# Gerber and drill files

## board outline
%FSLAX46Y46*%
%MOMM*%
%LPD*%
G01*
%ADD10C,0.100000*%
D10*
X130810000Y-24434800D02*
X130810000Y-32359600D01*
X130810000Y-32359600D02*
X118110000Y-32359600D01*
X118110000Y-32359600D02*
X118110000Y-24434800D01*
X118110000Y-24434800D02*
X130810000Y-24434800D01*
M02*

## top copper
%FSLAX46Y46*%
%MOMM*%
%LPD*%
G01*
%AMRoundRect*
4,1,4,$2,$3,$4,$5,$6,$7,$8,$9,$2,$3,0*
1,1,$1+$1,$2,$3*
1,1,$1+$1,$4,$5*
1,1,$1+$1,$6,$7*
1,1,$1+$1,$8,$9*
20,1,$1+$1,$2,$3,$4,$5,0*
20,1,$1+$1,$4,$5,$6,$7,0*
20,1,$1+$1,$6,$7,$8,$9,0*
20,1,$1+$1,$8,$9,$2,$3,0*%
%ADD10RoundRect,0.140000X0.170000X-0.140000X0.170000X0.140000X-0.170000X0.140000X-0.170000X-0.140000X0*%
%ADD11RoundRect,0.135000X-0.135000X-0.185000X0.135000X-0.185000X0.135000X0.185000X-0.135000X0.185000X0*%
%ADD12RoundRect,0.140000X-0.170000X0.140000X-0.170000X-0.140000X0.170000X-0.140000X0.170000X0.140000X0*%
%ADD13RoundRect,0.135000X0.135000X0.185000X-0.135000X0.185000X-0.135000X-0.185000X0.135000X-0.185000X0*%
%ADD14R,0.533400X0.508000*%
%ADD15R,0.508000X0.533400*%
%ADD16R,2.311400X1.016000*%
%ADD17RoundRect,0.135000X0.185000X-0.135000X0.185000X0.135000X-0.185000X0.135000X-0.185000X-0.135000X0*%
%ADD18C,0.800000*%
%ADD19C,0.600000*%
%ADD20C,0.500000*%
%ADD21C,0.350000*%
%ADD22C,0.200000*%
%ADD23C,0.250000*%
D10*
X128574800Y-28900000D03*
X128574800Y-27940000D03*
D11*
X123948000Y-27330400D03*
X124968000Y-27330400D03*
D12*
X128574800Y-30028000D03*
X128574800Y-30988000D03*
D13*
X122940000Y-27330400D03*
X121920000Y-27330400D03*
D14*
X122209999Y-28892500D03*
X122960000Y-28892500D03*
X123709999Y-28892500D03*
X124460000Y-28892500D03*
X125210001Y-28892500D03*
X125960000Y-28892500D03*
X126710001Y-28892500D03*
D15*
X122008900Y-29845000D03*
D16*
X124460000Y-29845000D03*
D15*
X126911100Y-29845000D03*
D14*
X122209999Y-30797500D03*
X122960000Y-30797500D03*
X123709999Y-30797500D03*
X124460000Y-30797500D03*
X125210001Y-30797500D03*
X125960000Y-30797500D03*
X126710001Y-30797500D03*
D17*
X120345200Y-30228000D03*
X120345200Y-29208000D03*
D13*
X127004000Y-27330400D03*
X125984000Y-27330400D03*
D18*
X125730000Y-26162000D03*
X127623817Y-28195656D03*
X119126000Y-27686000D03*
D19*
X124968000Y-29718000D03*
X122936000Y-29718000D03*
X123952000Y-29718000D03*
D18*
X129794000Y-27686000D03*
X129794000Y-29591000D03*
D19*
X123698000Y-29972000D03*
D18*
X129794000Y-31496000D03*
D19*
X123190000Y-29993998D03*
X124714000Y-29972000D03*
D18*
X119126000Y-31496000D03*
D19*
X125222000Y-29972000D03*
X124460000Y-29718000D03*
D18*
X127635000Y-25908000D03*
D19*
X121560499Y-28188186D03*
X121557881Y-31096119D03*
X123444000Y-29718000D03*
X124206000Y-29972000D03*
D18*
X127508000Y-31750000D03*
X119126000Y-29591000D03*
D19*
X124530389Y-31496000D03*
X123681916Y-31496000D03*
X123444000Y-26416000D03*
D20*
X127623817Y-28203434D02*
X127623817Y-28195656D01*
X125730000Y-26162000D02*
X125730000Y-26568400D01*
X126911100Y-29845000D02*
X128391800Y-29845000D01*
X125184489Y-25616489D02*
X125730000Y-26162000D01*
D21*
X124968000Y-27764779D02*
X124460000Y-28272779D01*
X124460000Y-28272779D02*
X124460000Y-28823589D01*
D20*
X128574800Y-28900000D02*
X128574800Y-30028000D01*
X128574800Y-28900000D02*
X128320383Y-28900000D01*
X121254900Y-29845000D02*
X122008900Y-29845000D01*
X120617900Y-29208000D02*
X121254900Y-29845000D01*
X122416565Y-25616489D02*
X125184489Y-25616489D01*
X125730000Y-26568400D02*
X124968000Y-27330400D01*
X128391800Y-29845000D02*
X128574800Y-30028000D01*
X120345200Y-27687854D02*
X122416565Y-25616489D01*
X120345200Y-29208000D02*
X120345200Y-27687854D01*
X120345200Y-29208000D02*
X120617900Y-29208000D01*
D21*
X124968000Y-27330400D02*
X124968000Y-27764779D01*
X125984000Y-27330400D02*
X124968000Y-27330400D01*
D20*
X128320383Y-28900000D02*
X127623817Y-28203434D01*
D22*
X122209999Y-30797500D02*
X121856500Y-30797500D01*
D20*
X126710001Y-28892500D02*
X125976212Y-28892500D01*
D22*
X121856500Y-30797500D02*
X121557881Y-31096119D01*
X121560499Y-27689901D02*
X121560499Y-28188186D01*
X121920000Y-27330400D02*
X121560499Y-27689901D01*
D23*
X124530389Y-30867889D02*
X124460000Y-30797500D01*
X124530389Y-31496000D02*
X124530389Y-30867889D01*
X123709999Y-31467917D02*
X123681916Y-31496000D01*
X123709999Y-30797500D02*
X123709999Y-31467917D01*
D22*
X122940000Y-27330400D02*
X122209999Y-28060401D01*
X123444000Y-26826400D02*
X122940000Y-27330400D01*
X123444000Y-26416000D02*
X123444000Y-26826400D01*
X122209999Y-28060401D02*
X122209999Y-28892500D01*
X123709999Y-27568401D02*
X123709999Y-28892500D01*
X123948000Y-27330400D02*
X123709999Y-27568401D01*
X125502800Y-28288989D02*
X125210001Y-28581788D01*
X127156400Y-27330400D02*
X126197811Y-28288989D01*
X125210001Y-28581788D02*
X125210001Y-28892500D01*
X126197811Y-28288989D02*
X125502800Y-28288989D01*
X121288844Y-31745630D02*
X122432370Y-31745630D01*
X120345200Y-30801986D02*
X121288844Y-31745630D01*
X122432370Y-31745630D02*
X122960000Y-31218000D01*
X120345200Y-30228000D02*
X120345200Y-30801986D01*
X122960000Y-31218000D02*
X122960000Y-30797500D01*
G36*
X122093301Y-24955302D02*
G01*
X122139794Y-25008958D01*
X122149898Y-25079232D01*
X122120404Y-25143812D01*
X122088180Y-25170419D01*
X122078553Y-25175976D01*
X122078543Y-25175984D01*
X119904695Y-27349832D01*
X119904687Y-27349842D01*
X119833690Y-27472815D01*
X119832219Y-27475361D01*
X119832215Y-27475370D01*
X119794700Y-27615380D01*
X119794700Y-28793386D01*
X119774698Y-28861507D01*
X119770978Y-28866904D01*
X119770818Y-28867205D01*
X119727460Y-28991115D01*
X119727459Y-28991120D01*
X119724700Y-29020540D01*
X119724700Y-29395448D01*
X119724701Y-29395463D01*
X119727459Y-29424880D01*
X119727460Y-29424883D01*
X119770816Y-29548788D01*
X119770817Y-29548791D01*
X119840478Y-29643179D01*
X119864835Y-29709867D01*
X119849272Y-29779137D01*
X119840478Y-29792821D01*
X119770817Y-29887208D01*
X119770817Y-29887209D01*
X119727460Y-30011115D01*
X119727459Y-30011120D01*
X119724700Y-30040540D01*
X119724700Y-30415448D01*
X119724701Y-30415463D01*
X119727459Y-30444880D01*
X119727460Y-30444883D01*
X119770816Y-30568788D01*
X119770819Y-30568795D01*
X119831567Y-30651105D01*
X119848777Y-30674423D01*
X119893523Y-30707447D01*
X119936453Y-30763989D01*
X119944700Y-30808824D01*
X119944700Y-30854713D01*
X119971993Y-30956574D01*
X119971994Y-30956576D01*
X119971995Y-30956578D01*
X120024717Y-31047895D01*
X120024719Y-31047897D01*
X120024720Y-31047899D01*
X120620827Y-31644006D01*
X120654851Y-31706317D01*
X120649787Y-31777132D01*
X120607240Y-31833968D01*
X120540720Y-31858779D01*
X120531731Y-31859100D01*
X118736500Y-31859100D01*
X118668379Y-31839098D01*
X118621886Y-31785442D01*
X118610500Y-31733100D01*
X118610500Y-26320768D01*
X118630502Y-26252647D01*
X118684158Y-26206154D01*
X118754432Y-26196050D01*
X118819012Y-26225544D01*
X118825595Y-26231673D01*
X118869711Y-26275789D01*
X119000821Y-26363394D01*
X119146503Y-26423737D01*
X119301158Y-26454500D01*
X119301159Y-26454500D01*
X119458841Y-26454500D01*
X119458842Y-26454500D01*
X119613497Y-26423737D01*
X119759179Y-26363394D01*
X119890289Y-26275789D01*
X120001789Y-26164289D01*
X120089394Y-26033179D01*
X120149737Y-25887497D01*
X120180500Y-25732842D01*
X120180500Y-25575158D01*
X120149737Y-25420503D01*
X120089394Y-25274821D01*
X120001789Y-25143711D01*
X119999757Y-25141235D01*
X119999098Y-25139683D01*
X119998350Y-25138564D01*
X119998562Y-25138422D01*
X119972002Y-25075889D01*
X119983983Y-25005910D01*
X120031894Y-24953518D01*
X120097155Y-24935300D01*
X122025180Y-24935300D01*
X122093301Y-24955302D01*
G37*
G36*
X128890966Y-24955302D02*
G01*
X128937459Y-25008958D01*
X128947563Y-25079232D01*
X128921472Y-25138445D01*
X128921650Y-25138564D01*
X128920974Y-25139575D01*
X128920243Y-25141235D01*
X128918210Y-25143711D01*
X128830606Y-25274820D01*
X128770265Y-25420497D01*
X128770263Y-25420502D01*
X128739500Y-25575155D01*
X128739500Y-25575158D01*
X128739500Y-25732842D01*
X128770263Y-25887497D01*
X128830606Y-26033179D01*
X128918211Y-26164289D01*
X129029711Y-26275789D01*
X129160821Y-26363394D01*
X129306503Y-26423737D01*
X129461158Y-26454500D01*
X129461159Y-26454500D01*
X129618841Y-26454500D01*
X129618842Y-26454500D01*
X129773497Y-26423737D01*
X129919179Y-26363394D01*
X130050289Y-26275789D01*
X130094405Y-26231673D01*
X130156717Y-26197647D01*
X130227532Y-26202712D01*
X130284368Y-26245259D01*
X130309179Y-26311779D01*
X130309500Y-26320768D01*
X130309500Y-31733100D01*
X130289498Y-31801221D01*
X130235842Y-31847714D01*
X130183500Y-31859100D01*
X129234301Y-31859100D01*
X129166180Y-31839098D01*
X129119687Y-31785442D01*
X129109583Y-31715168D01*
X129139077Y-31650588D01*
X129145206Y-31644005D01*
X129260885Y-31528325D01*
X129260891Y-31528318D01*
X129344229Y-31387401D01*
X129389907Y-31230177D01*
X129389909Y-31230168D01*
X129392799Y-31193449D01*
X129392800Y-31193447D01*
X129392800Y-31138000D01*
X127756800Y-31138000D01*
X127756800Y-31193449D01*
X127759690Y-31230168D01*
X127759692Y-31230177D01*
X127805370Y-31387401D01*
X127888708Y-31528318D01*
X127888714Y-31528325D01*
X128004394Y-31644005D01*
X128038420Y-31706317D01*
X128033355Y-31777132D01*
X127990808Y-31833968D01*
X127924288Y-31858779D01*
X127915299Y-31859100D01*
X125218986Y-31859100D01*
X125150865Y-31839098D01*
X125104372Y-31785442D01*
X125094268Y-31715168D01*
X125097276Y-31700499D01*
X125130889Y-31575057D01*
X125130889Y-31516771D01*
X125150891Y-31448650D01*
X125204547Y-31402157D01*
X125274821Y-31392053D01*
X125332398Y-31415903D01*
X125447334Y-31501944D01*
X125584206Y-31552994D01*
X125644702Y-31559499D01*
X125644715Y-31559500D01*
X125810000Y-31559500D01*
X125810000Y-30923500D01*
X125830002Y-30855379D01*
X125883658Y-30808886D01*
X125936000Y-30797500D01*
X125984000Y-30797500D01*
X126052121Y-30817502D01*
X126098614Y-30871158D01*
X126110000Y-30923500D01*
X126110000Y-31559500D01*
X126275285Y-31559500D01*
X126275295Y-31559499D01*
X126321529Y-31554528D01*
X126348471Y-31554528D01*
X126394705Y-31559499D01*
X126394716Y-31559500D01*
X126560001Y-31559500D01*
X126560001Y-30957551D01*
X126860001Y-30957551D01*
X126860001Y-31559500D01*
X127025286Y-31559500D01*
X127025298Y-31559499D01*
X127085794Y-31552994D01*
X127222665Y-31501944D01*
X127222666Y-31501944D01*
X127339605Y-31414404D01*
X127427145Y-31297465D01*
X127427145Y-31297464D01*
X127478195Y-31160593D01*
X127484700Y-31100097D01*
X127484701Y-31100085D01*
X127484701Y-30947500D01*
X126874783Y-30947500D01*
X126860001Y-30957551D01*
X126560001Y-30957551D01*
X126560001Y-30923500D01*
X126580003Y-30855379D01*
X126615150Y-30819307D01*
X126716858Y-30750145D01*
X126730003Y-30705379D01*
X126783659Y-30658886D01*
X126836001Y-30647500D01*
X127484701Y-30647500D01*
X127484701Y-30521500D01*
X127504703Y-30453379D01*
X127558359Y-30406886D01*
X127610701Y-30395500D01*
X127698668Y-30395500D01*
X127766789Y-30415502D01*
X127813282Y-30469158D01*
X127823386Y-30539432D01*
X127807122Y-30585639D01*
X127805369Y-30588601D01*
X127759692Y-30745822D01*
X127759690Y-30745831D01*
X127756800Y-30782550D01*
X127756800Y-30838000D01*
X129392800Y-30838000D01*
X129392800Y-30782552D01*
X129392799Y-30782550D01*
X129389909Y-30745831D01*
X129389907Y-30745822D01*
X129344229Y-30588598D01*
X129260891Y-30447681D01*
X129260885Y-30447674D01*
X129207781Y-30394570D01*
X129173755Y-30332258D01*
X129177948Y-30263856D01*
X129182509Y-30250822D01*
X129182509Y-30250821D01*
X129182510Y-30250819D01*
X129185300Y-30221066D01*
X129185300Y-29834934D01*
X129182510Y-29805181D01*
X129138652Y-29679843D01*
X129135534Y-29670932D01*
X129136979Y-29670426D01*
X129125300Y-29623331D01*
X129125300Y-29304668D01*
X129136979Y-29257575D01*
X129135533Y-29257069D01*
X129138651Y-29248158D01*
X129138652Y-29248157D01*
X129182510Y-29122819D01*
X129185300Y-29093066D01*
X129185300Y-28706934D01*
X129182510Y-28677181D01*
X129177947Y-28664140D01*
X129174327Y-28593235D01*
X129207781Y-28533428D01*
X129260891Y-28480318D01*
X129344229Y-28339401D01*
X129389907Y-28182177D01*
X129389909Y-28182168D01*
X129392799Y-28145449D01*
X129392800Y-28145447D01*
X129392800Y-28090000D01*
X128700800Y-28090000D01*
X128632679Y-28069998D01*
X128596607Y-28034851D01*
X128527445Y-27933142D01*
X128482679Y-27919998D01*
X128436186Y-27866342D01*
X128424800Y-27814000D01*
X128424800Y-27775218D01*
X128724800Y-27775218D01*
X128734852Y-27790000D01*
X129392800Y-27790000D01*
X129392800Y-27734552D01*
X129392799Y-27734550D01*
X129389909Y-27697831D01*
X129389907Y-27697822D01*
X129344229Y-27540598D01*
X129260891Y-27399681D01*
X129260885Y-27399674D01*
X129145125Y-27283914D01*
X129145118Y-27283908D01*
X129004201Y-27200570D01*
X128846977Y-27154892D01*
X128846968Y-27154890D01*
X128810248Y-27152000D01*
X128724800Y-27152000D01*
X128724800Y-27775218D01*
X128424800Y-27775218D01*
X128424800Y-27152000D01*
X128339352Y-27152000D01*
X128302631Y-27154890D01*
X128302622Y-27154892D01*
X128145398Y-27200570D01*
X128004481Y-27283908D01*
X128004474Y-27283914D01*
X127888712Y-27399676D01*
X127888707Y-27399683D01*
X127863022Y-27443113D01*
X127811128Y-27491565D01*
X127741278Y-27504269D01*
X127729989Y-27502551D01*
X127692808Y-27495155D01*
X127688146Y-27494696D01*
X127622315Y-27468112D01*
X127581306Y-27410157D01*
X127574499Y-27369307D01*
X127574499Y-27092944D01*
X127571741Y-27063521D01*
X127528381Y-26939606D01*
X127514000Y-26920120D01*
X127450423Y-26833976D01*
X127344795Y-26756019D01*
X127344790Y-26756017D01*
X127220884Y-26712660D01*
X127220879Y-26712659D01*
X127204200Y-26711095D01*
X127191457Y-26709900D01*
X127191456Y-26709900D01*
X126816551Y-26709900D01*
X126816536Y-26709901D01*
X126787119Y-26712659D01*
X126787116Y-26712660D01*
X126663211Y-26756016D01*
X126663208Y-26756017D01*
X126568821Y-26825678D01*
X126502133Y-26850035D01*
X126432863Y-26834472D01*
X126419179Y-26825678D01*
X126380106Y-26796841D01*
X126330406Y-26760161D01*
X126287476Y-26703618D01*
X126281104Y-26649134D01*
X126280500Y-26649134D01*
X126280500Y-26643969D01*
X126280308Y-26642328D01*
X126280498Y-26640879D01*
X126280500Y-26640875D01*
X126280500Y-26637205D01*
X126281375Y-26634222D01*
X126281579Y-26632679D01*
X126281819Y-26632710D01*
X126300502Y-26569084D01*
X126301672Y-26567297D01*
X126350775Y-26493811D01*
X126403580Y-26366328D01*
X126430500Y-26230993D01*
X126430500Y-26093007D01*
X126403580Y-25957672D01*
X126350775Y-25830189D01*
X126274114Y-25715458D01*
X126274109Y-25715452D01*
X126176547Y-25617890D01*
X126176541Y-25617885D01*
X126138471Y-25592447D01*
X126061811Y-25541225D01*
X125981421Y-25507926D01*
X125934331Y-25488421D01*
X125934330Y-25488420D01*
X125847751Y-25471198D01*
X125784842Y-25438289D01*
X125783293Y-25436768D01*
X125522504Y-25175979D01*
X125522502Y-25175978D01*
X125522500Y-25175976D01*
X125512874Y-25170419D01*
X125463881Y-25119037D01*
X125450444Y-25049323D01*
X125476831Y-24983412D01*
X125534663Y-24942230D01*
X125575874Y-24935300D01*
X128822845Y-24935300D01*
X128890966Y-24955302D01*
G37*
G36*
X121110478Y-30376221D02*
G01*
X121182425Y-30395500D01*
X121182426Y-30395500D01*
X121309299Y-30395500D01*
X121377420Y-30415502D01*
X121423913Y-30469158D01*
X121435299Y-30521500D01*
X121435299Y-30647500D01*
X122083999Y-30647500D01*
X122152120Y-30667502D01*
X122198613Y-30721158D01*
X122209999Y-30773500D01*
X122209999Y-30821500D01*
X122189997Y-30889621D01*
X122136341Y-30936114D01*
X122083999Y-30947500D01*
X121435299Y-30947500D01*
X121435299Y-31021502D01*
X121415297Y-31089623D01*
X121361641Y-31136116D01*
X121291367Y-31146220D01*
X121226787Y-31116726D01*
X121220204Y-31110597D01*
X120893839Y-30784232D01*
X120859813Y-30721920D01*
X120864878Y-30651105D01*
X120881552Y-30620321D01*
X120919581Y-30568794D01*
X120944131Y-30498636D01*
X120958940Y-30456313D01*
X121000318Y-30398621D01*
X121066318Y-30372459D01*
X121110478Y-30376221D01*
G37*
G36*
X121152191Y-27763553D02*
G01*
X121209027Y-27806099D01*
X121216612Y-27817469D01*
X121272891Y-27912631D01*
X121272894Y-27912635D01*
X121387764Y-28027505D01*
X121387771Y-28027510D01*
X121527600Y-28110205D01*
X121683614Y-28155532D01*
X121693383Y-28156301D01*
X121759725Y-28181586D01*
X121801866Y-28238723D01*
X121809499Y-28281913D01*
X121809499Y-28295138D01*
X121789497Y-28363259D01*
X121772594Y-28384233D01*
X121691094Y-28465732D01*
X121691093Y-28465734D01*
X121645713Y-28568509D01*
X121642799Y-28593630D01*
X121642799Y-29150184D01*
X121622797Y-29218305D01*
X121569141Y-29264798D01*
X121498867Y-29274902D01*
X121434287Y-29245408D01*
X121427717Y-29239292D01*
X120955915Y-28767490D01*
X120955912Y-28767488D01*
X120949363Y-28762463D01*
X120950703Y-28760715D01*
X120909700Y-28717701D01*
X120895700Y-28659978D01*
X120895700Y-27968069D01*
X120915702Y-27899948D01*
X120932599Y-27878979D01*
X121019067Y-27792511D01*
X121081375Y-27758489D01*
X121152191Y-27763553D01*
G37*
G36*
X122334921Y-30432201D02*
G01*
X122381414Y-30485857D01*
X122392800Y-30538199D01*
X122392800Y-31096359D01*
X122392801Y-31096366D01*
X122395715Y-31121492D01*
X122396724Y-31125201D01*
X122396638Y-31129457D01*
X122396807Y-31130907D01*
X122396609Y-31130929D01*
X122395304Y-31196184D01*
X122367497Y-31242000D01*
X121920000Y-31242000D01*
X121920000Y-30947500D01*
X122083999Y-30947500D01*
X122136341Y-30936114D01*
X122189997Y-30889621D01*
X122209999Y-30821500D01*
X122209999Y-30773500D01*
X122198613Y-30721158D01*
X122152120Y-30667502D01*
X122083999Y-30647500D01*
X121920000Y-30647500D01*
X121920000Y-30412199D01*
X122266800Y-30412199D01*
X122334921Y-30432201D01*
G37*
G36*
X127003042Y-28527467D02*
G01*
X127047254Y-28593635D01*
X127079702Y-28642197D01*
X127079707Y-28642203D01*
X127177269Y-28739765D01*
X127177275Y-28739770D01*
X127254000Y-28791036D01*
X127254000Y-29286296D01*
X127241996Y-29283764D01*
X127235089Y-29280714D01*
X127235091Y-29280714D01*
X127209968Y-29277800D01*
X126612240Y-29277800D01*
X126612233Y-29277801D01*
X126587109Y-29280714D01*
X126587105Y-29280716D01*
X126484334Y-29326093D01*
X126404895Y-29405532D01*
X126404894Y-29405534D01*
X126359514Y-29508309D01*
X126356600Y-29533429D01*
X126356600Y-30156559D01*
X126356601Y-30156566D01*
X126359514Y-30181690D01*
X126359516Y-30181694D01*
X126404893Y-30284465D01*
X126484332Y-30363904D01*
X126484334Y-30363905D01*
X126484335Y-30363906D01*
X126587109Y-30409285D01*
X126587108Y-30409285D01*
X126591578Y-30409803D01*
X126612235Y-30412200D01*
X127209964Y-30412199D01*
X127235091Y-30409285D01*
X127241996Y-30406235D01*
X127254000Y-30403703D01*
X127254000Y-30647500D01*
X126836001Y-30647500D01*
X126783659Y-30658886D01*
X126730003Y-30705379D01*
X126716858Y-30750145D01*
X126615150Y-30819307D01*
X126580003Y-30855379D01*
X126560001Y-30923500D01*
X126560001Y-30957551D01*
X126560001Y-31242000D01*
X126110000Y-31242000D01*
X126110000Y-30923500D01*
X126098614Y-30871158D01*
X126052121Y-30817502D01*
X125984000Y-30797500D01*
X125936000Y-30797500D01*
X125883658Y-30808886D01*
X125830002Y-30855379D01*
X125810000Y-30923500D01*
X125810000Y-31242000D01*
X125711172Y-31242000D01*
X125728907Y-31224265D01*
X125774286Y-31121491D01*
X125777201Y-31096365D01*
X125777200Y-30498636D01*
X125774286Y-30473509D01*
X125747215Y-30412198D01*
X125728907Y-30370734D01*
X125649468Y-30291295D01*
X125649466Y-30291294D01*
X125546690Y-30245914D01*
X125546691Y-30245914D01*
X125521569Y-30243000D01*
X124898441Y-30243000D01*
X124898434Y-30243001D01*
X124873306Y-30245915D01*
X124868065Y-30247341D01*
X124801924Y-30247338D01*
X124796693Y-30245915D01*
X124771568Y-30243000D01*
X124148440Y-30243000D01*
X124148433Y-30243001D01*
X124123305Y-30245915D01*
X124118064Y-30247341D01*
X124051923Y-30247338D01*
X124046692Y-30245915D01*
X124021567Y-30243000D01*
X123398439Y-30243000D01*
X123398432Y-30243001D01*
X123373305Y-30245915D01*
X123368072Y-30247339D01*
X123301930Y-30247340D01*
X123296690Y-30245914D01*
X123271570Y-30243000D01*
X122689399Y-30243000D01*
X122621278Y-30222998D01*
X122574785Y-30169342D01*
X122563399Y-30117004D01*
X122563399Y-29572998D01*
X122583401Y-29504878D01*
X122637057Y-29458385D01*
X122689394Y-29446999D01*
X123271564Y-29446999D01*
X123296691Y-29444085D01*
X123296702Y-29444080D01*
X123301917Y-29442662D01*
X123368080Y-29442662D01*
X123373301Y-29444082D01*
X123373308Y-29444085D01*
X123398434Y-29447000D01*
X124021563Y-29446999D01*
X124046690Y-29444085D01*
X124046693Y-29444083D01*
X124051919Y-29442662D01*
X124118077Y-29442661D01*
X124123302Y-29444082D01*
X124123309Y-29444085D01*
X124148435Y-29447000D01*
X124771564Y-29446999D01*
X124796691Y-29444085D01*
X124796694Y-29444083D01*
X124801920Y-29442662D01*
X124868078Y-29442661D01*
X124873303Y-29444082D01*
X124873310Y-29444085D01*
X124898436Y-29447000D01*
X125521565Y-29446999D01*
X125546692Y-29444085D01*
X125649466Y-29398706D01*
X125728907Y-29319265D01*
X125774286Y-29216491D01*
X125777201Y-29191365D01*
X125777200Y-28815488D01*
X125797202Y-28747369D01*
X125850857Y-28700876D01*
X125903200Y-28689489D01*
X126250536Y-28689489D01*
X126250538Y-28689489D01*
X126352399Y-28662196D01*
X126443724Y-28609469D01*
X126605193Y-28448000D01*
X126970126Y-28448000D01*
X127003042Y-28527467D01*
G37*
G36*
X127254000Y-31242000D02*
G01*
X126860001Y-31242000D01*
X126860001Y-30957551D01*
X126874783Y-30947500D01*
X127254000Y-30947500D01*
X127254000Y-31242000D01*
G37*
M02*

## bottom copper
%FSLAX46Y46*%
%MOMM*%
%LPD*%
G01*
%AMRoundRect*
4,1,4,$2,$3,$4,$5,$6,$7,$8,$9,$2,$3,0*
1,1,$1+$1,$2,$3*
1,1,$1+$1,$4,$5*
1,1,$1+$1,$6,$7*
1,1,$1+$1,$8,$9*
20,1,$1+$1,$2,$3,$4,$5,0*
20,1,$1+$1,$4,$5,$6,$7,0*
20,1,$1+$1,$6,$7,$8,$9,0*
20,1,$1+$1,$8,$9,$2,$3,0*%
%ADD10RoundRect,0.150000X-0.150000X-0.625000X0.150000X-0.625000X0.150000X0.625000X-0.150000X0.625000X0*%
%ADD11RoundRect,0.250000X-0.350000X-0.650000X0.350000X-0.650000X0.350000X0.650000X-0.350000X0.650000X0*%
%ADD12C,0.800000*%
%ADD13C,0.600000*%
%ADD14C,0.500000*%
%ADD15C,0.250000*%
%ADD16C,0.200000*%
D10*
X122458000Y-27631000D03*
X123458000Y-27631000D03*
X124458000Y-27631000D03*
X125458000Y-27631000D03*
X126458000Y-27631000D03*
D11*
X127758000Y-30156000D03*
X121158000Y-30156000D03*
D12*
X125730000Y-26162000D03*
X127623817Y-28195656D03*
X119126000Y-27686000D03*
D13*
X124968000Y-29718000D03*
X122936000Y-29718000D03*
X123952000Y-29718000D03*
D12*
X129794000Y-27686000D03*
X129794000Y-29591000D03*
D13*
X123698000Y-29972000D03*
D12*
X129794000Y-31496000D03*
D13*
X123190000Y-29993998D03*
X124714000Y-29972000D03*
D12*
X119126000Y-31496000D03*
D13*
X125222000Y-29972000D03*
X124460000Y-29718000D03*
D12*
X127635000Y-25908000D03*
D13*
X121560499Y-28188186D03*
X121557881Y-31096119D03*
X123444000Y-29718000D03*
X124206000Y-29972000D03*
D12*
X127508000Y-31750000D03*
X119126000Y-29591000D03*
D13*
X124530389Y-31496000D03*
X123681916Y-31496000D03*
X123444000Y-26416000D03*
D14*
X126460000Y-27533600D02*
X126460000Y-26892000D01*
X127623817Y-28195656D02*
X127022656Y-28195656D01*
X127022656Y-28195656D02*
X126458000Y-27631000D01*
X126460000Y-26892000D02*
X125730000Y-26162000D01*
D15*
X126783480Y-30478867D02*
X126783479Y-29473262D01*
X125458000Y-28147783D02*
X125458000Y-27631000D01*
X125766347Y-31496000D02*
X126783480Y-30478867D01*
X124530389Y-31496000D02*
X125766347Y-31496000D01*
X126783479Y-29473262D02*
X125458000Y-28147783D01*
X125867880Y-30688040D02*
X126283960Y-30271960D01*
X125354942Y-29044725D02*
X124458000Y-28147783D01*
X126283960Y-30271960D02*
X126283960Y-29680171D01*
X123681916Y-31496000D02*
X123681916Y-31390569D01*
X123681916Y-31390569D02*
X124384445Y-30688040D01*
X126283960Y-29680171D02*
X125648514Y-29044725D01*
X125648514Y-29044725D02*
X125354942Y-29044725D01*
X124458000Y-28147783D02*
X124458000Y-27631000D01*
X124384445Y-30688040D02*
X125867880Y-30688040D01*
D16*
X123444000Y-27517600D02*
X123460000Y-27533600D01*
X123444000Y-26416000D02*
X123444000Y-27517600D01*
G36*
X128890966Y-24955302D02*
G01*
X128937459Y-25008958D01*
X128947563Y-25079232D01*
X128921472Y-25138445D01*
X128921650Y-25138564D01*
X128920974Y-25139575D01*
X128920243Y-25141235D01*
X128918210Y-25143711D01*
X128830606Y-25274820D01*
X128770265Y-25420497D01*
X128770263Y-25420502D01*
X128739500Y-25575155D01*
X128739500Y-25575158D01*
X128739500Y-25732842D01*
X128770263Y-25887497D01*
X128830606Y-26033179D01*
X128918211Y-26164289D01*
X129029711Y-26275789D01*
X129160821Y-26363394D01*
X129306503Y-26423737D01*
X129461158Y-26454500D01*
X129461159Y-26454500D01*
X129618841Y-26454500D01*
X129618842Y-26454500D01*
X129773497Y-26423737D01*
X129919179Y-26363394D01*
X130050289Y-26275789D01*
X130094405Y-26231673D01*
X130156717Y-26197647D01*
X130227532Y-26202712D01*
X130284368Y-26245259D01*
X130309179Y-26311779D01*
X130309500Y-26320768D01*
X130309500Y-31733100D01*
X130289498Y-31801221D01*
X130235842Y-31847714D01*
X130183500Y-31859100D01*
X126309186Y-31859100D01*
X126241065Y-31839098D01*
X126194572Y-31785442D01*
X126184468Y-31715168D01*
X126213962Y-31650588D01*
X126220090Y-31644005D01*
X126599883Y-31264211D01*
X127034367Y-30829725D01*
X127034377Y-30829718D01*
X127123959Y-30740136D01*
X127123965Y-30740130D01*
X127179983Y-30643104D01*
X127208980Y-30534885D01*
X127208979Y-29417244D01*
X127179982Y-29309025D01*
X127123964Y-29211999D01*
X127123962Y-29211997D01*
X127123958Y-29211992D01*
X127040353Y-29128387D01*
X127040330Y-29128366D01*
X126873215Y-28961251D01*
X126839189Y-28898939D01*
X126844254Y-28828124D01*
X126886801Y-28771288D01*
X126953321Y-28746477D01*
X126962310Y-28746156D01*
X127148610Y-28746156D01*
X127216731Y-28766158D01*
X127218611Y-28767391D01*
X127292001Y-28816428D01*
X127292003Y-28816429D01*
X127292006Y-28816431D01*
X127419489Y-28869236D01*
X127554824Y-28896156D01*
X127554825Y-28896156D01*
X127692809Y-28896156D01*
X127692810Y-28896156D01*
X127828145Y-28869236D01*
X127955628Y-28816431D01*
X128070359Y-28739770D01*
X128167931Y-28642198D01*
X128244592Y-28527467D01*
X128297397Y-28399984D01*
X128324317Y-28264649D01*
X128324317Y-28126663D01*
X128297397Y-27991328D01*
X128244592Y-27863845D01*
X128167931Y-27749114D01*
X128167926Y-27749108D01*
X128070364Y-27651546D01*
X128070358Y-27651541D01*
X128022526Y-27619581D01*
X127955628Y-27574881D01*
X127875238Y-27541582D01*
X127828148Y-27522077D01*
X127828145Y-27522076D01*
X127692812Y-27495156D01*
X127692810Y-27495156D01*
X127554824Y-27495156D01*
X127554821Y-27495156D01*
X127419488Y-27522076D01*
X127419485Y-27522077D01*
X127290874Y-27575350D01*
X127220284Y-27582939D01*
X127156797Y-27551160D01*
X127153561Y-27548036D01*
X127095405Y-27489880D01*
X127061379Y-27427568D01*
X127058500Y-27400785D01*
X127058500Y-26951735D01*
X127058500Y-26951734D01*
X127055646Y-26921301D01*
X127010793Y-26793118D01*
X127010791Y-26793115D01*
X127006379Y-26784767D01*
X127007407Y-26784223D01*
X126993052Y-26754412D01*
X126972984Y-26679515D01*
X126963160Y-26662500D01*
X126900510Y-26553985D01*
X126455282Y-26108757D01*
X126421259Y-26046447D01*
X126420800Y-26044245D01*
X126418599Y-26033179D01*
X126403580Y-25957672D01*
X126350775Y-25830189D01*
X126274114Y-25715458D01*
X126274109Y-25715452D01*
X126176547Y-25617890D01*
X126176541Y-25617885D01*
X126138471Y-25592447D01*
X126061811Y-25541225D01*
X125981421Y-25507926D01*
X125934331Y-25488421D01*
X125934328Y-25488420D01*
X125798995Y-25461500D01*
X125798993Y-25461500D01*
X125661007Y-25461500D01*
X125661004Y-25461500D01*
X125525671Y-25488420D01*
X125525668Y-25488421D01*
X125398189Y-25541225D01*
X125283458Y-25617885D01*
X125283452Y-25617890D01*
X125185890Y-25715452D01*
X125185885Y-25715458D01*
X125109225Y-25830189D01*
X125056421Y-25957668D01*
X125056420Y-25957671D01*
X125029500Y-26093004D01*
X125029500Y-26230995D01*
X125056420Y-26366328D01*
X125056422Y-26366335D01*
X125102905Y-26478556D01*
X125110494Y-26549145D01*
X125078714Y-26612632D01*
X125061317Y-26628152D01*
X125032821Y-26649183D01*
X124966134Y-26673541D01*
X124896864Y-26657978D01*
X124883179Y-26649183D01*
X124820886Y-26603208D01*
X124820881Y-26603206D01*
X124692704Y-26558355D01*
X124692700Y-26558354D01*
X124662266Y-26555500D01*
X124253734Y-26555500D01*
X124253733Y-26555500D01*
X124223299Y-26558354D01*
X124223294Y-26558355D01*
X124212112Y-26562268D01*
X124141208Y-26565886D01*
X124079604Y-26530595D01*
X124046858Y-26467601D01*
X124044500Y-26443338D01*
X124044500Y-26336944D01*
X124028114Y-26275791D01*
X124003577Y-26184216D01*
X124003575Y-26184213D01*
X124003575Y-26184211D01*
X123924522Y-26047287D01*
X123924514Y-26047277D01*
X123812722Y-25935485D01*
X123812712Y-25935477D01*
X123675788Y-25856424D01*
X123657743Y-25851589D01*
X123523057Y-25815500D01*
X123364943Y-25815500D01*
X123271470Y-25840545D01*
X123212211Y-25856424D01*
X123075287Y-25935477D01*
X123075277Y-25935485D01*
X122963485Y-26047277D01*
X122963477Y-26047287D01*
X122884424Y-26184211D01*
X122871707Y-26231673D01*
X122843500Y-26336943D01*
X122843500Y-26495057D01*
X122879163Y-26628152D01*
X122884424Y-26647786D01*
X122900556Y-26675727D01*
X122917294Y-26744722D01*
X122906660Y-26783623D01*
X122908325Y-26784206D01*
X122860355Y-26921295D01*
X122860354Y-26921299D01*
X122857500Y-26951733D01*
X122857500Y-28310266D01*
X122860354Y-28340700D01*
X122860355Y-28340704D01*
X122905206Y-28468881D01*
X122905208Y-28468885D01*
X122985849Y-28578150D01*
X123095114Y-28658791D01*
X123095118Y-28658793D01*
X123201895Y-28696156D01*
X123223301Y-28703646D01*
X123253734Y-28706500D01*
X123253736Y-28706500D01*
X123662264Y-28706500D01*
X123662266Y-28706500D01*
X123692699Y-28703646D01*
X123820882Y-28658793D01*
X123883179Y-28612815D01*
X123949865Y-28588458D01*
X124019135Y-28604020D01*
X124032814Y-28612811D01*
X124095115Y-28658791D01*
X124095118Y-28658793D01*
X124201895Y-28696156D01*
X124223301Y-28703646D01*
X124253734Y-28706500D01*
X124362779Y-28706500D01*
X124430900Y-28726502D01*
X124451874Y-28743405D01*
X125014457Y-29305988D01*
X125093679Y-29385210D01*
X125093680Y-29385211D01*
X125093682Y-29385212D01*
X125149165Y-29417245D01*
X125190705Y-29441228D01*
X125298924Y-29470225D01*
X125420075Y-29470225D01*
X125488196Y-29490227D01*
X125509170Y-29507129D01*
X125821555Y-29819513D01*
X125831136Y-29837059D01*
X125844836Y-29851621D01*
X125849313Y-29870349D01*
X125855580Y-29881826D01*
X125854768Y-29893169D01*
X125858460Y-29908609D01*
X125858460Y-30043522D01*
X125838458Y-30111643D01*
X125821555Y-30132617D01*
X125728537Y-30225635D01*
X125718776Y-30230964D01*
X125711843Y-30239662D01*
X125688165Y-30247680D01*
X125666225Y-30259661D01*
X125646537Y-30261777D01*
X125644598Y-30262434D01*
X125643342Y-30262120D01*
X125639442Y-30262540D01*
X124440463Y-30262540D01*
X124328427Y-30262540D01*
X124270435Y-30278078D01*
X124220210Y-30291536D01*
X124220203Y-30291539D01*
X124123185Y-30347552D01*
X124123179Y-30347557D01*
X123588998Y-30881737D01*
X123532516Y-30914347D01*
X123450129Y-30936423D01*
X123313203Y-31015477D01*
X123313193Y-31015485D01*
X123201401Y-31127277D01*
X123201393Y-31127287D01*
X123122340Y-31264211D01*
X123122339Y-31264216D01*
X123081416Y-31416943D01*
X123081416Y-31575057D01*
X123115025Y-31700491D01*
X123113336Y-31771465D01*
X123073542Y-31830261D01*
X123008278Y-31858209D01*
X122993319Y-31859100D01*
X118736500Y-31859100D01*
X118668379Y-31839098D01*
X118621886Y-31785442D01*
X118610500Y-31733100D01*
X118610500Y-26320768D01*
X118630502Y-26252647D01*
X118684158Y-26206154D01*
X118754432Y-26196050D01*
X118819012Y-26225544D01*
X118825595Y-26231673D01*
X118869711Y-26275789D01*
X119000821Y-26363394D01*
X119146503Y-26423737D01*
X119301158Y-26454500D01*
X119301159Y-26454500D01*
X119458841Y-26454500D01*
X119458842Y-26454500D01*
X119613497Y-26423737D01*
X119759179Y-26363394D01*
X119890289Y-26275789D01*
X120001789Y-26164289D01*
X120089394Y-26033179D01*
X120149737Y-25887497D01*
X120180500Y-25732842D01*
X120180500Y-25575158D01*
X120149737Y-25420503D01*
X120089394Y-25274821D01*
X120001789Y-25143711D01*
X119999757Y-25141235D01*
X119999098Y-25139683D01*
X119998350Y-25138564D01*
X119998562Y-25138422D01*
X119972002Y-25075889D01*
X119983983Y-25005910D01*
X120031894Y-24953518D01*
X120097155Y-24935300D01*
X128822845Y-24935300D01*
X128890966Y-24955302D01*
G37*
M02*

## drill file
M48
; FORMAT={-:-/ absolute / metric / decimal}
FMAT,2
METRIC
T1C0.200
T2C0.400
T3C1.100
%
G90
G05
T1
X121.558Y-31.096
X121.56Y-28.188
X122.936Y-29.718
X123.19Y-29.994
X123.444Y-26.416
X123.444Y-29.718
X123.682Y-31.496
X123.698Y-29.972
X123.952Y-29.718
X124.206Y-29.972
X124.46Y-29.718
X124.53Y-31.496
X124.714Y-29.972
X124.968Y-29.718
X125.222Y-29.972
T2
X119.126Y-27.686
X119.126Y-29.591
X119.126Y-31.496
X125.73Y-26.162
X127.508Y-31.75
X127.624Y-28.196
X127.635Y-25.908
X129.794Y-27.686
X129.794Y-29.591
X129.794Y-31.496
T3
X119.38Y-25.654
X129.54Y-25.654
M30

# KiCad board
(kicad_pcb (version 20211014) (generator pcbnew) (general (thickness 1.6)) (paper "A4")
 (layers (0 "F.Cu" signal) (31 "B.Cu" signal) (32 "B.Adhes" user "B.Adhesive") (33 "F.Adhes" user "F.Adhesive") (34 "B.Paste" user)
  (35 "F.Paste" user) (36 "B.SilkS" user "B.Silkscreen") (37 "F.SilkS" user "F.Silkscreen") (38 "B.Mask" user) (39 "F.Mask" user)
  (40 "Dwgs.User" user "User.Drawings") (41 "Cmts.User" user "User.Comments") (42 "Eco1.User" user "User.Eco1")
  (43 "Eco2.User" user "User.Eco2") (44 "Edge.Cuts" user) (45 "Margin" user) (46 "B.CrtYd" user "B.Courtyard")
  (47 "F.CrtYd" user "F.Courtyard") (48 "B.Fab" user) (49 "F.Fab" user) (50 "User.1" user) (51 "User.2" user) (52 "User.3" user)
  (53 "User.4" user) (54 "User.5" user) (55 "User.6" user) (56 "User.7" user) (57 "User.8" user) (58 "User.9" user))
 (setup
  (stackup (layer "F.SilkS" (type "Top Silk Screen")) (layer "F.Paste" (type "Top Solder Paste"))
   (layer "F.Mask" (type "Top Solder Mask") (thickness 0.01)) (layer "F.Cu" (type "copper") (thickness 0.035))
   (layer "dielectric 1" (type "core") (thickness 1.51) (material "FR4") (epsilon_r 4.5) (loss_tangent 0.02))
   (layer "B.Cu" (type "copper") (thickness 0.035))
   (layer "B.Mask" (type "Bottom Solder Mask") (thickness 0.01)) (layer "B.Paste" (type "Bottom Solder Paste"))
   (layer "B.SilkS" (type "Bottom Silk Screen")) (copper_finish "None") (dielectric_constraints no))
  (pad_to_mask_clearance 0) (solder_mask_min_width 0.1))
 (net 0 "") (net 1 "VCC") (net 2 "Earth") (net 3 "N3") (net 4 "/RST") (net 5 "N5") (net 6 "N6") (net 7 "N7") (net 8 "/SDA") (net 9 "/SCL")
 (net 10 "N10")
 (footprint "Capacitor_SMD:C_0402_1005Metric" (layer "F.Cu") (at 128.5748 28.42 90)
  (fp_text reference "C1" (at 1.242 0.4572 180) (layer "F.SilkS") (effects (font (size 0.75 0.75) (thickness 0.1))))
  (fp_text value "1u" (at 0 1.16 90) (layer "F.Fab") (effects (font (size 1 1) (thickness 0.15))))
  (pad "1" smd roundrect (at -0.48 0 90) (size 0.56 0.62) (layers "F.Cu" "F.Paste" "F.Mask") (roundrect_rratio 0.25) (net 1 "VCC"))
  (pad "2" smd roundrect (at 0.48 0 90) (size 0.56 0.62) (layers "F.Cu" "F.Paste" "F.Mask") (roundrect_rratio 0.25) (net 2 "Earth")))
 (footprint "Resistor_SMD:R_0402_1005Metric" (layer "F.Cu") (at 124.458 27.3304)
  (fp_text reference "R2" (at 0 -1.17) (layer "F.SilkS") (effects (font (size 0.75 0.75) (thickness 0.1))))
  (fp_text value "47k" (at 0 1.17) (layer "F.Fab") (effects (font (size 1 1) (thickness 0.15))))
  (pad "1" smd roundrect (at -0.51 0) (size 0.54 0.64) (layers "F.Cu" "F.Paste" "F.Mask") (roundrect_rratio 0.25) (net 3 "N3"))
  (pad "2" smd roundrect (at 0.51 0) (size 0.54 0.64) (layers "F.Cu" "F.Paste" "F.Mask") (roundrect_rratio 0.25) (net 1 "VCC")))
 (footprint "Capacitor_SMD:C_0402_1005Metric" (layer "F.Cu") (at 128.5748 30.508 -90)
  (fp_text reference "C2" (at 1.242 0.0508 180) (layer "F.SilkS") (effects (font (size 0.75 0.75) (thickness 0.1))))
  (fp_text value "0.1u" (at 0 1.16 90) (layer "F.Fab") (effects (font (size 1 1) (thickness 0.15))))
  (pad "1" smd roundrect (at -0.48 0 270) (size 0.56 0.62) (layers "F.Cu" "F.Paste" "F.Mask") (roundrect_rratio 0.25) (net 1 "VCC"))
  (pad "2" smd roundrect (at 0.48 0 270) (size 0.56 0.62) (layers "F.Cu" "F.Paste" "F.Mask") (roundrect_rratio 0.25) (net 2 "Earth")))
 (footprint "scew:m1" (layer "F.Cu") (at 119.38 25.654 180)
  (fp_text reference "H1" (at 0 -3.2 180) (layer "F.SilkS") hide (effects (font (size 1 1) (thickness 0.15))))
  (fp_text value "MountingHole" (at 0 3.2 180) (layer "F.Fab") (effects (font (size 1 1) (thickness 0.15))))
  (pad "" np_thru_hole circle (at 0 0 180) (size 1 1) (drill 1.1) (layers F&B.Cu *.Mask)))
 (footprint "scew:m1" (layer "F.Cu") (at 129.54 25.654)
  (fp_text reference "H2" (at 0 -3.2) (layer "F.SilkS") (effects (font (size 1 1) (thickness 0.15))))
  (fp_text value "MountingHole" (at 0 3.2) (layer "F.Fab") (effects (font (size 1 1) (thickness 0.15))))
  (pad "" np_thru_hole circle (at 0 0) (size 1 1) (drill 1.1) (layers F&B.Cu *.Mask)))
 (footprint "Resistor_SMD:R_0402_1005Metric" (layer "F.Cu") (at 122.43 27.3304 180)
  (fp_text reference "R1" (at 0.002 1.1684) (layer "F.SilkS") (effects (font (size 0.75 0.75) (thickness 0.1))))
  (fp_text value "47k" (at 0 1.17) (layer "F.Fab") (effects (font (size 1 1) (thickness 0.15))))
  (pad "1" smd roundrect (at -0.51 0 180) (size 0.54 0.64) (layers "F.Cu" "F.Paste" "F.Mask") (roundrect_rratio 0.25) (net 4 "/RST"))
  (pad "2" smd roundrect (at 0.51 0 180) (size 0.54 0.64) (layers "F.Cu" "F.Paste" "F.Mask") (roundrect_rratio 0.25) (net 2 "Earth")))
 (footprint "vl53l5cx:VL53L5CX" (layer "F.Cu") (at 124.46 29.845)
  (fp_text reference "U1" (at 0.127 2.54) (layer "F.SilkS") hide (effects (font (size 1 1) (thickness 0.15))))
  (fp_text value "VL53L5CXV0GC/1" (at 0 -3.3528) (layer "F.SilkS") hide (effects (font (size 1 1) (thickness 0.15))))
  (pad "A1" smd rect (at -2.250001 -0.9525) (size 0.5334 0.508) (layers "F.Cu" "F.Paste" "F.Mask") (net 4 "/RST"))
  (pad "A2" smd rect (at -1.5 -0.9525) (size 0.5334 0.508) (layers "F.Cu" "F.Paste" "F.Mask") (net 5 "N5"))
  (pad "A3" smd rect (at -0.750001 -0.9525) (size 0.5334 0.508) (layers "F.Cu" "F.Paste" "F.Mask") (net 3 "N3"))
  (pad "A4" smd rect (at 0 -0.9525) (size 0.5334 0.508) (layers "F.Cu" "F.Paste" "F.Mask") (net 1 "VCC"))
  (pad "A5" smd rect (at 0.750001 -0.9525) (size 0.5334 0.508) (layers "F.Cu" "F.Paste" "F.Mask") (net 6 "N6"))
  (pad "A6" smd rect (at 1.5 -0.9525) (size 0.5334 0.508) (layers "F.Cu" "F.Paste" "F.Mask") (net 2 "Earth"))
  (pad "A7" smd rect (at 2.250001 -0.9525) (size 0.5334 0.508) (layers "F.Cu" "F.Paste" "F.Mask") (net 2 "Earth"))
  (pad "B1" smd rect (at -2.4511 0 90) (size 0.5334 0.508) (layers "F.Cu" "F.Paste" "F.Mask") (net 1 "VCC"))
  (pad "B4" smd rect (at 0 0) (size 2.3114 1.016) (layers "F.Cu" "F.Paste" "F.Mask") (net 2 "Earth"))
  (pad "B7" smd rect (at 2.4511 0 90) (size 0.5334 0.508) (layers "F.Cu" "F.Paste" "F.Mask") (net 1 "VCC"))
  (pad "C1" smd rect (at -2.250001 0.9525) (size 0.5334 0.508) (layers "F.Cu" "F.Paste" "F.Mask") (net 2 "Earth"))
  (pad "C2" smd rect (at -1.5 0.9525) (size 0.5334 0.508) (layers "F.Cu" "F.Paste" "F.Mask") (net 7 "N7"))
  (pad "C3" smd rect (at -0.750001 0.9525) (size 0.5334 0.508) (layers "F.Cu" "F.Paste" "F.Mask") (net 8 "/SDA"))
  (pad "C4" smd rect (at 0 0.9525) (size 0.5334 0.508) (layers "F.Cu" "F.Paste" "F.Mask") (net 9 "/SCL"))
  (pad "C5" smd rect (at 0.750001 0.9525) (size 0.5334 0.508) (layers "F.Cu" "F.Paste" "F.Mask") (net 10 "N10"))
  (pad "C6" smd rect (at 1.5 0.9525) (size 0.5334 0.508) (layers "F.Cu" "F.Paste" "F.Mask") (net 2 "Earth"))
  (pad "C7" smd rect (at 2.250001 0.9525) (size 0.5334 0.508) (layers "F.Cu" "F.Paste" "F.Mask") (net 2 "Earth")))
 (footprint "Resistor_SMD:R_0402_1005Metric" (layer "F.Cu") (at 120.3452 29.718 90)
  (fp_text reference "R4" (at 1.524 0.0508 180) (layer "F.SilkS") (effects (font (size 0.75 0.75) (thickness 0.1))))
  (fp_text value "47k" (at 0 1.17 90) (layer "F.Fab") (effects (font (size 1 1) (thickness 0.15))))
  (pad "1" smd roundrect (at -0.51 0 90) (size 0.54 0.64) (layers "F.Cu" "F.Paste" "F.Mask") (roundrect_rratio 0.25) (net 7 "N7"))
  (pad "2" smd roundrect (at 0.51 0 90) (size 0.54 0.64) (layers "F.Cu" "F.Paste" "F.Mask") (roundrect_rratio 0.25) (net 1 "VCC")))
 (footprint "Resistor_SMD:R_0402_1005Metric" (layer "F.Cu") (at 126.494 27.3304 180)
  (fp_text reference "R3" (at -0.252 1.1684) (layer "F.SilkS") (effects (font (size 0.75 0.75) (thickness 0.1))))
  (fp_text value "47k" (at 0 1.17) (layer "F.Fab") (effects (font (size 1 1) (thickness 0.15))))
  (pad "1" smd roundrect (at -0.51 0 180) (size 0.54 0.64) (layers "F.Cu" "F.Paste" "F.Mask") (roundrect_rratio 0.25) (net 6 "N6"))
  (pad "2" smd roundrect (at 0.51 0 180) (size 0.54 0.64) (layers "F.Cu" "F.Paste" "F.Mask") (roundrect_rratio 0.25) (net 1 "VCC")))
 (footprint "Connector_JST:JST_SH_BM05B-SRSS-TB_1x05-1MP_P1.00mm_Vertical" (layer "B.Cu") (at 124.458 28.956)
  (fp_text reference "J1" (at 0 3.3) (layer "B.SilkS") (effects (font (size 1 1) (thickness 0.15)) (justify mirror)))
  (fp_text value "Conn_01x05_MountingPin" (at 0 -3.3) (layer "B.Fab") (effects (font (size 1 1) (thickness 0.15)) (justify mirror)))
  (pad "1" smd roundrect (at -2 -1.325) (size 0.6 1.55) (layers "B.Cu" "B.Paste" "B.Mask") (roundrect_rratio 0.25) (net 2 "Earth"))
  (pad "2" smd roundrect (at -1 -1.325) (size 0.6 1.55) (layers "B.Cu" "B.Paste" "B.Mask") (roundrect_rratio 0.25) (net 4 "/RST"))
  (pad "3" smd roundrect (at 0 -1.325) (size 0.6 1.55) (layers "B.Cu" "B.Paste" "B.Mask") (roundrect_rratio 0.25) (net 8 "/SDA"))
  (pad "4" smd roundrect (at 1 -1.325) (size 0.6 1.55) (layers "B.Cu" "B.Paste" "B.Mask") (roundrect_rratio 0.25) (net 9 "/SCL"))
  (pad "5" smd roundrect (at 2 -1.325) (size 0.6 1.55) (layers "B.Cu" "B.Paste" "B.Mask") (roundrect_rratio 0.25) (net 1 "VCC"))
  (pad "MP" smd roundrect (at 3.3 1.2) (size 1.2 1.8) (layers "B.Cu" "B.Paste" "B.Mask") (roundrect_rratio 0.208333) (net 2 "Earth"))
  (pad "MP" smd roundrect (at -3.3 1.2) (size 1.2 1.8) (layers "B.Cu" "B.Paste" "B.Mask") (roundrect_rratio 0.208333) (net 2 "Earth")))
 (gr_line (start 130.81 24.4348) (end 130.81 32.3596) (layer "Edge.Cuts") (width 0.1))
 (gr_line (start 130.81 32.3596) (end 118.11 32.3596) (layer "Edge.Cuts") (width 0.1))
 (gr_line (start 118.11 32.3596) (end 118.11 24.4348) (layer "Edge.Cuts") (width 0.1))
 (gr_line (start 118.11 24.4348) (end 130.81 24.4348) (layer "Edge.Cuts") (width 0.1))
 (segment (start 127.623817 28.203434) (end 127.623817 28.195656) (width 0.5) (layer "F.Cu") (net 1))
 (segment (start 125.73 26.162) (end 125.73 26.5684) (width 0.5) (layer "F.Cu") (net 1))
 (segment (start 126.9111 29.845) (end 128.3918 29.845) (width 0.5) (layer "F.Cu") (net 1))
 (segment (start 125.184489 25.616489) (end 125.73 26.162) (width 0.5) (layer "F.Cu") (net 1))
 (segment (start 124.968 27.764779) (end 124.46 28.272779) (width 0.35) (layer "F.Cu") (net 1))
 (segment (start 124.46 28.272779) (end 124.46 28.823589) (width 0.35) (layer "F.Cu") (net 1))
 (segment (start 128.5748 28.9) (end 128.5748 30.028) (width 0.5) (layer "F.Cu") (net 1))
 (segment (start 128.5748 28.9) (end 128.320383 28.9) (width 0.5) (layer "F.Cu") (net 1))
 (segment (start 121.2549 29.845) (end 122.0089 29.845) (width 0.5) (layer "F.Cu") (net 1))
 (segment (start 120.6179 29.208) (end 121.2549 29.845) (width 0.5) (layer "F.Cu") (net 1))
 (segment (start 122.416565 25.616489) (end 125.184489 25.616489) (width 0.5) (layer "F.Cu") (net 1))
 (segment (start 125.73 26.5684) (end 124.968 27.3304) (width 0.5) (layer "F.Cu") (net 1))
 (segment (start 128.3918 29.845) (end 128.5748 30.028) (width 0.5) (layer "F.Cu") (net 1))
 (segment (start 120.3452 27.687854) (end 122.416565 25.616489) (width 0.5) (layer "F.Cu") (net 1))
 (segment (start 120.3452 29.208) (end 120.3452 27.687854) (width 0.5) (layer "F.Cu") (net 1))
 (segment (start 120.3452 29.208) (end 120.6179 29.208) (width 0.5) (layer "F.Cu") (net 1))
 (segment (start 124.968 27.3304) (end 124.968 27.764779) (width 0.35) (layer "F.Cu") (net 1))
 (segment (start 125.984 27.3304) (end 124.968 27.3304) (width 0.35) (layer "F.Cu") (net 1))
 (segment (start 128.320383 28.9) (end 127.623817 28.203434) (width 0.5) (layer "F.Cu") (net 1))
 (via (at 125.73 26.162) (size 0.8) (drill 0.4) (layers "F.Cu" "B.Cu") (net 1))
 (via (at 127.623817 28.195656) (size 0.8) (drill 0.4) (layers "F.Cu" "B.Cu") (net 1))
 (segment (start 126.46 27.5336) (end 126.46 26.892) (width 0.5) (layer "B.Cu") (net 1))
 (segment (start 127.623817 28.195656) (end 127.022656 28.195656) (width 0.5) (layer "B.Cu") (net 1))
 (segment (start 127.022656 28.195656) (end 126.458 27.631) (width 0.5) (layer "B.Cu") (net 1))
 (segment (start 126.46 26.892) (end 125.73 26.162) (width 0.5) (layer "B.Cu") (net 1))
 (segment (start 122.209999 30.7975) (end 121.8565 30.7975) (width 0.2) (layer "F.Cu") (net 2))
 (segment (start 126.710001 28.8925) (end 125.976212 28.8925) (width 0.5) (layer "F.Cu") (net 2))
 (segment (start 121.8565 30.7975) (end 121.557881 31.096119) (width 0.2) (layer "F.Cu") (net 2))
 (segment (start 121.560499 27.689901) (end 121.560499 28.188186) (width 0.2) (layer "F.Cu") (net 2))
 (segment (start 121.92 27.3304) (end 121.560499 27.689901) (width 0.2) (layer "F.Cu") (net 2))
 (via (at 119.126 27.686) (size 0.8) (drill 0.4) (layers "F.Cu" "B.Cu") (free) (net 2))
 (via (at 124.968 29.718) (size 0.6) (drill 0.2) (layers "F.Cu" "B.Cu") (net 2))
 (via (at 122.936 29.718) (size 0.6) (drill 0.2) (layers "F.Cu" "B.Cu") (free) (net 2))
 (via (at 123.952 29.718) (size 0.6) (drill 0.2) (layers "F.Cu" "B.Cu") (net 2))
 (via (at 129.794 27.686) (size 0.8) (drill 0.4) (layers "F.Cu" "B.Cu") (free) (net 2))
 (via (at 129.794 29.591) (size 0.8) (drill 0.4) (layers "F.Cu" "B.Cu") (free) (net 2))
 (via (at 123.698 29.972) (size 0.6) (drill 0.2) (layers "F.Cu" "B.Cu") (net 2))
 (via (at 129.794 31.496) (size 0.8) (drill 0.4) (layers "F.Cu" "B.Cu") (free) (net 2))
 (via (at 123.19 29.993998) (size 0.6) (drill 0.2) (layers "F.Cu" "B.Cu") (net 2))
 (via (at 124.714 29.972) (size 0.6) (drill 0.2) (layers "F.Cu" "B.Cu") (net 2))
 (via (at 119.126 31.496) (size 0.8) (drill 0.4) (layers "F.Cu" "B.Cu") (free) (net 2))
 (via (at 125.222 29.972) (size 0.6) (drill 0.2) (layers "F.Cu" "B.Cu") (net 2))
 (via (at 124.46 29.718) (size 0.6) (drill 0.2) (layers "F.Cu" "B.Cu") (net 2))
 (via (at 127.635 25.908) (size 0.8) (drill 0.4) (layers "F.Cu" "B.Cu") (free) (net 2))
 (via (at 121.560499 28.188186) (size 0.6) (drill 0.2) (layers "F.Cu" "B.Cu") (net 2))
 (via (at 121.557881 31.096119) (size 0.6) (drill 0.2) (layers "F.Cu" "B.Cu") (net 2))
 (via (at 123.444 29.718) (size 0.6) (drill 0.2) (layers "F.Cu" "B.Cu") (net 2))
 (via (at 124.206 29.972) (size 0.6) (drill 0.2) (layers "F.Cu" "B.Cu") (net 2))
 (via (at 127.508 31.75) (size 0.8) (drill 0.4) (layers "F.Cu" "B.Cu") (free) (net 2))
 (via (at 119.126 29.591) (size 0.8) (drill 0.4) (layers "F.Cu" "B.Cu") (free) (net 2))
 (segment (start 124.530389 30.867889) (end 124.46 30.7975) (width 0.25) (layer "F.Cu") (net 9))
 (segment (start 124.530389 31.496) (end 124.530389 30.867889) (width 0.25) (layer "F.Cu") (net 9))
 (via (at 124.530389 31.496) (size 0.6) (drill 0.2) (layers "F.Cu" "B.Cu") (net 9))
 (segment (start 126.78348 30.478867) (end 126.783479 29.473262) (width 0.25) (layer "B.Cu") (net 9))
 (segment (start 125.458 28.147783) (end 125.458 27.631) (width 0.25) (layer "B.Cu") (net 9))
 (segment (start 125.766347 31.496) (end 126.78348 30.478867) (width 0.25) (layer "B.Cu") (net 9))
 (segment (start 124.530389 31.496) (end 125.766347 31.496) (width 0.25) (layer "B.Cu") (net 9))
 (segment (start 126.783479 29.473262) (end 125.458 28.147783) (width 0.25) (layer "B.Cu") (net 9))
 (segment (start 123.709999 31.467917) (end 123.681916 31.496) (width 0.25) (layer "F.Cu") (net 8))
 (segment (start 123.709999 30.7975) (end 123.709999 31.467917) (width 0.25) (layer "F.Cu") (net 8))
 (via (at 123.681916 31.496) (size 0.6) (drill 0.2) (layers "F.Cu" "B.Cu") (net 8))
 (segment (start 125.86788 30.68804) (end 126.28396 30.27196) (width 0.25) (layer "B.Cu") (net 8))
 (segment (start 125.354942 29.044725) (end 124.458 28.147783) (width 0.25) (layer "B.Cu") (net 8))
 (segment (start 126.28396 30.27196) (end 126.28396 29.680171) (width 0.25) (layer "B.Cu") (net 8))
 (segment (start 123.681916 31.496) (end 123.681916 31.390569) (width 0.25) (layer "B.Cu") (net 8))
 (segment (start 123.681916 31.390569) (end 124.384445 30.68804) (width 0.25) (layer "B.Cu") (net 8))
 (segment (start 126.28396 29.680171) (end 125.648514 29.044725) (width 0.25) (layer "B.Cu") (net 8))
 (segment (start 125.648514 29.044725) (end 125.354942 29.044725) (width 0.25) (layer "B.Cu") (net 8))
 (segment (start 124.458 28.147783) (end 124.458 27.631) (width 0.25) (layer "B.Cu") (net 8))
 (segment (start 124.384445 30.68804) (end 125.86788 30.68804) (width 0.25) (layer "B.Cu") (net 8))
 (segment (start 122.94 27.3304) (end 122.209999 28.060401) (width 0.2) (layer "F.Cu") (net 4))
 (segment (start 123.444 26.8264) (end 122.94 27.3304) (width 0.2) (layer "F.Cu") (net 4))
 (segment (start 123.444 26.416) (end 123.444 26.8264) (width 0.2) (layer "F.Cu") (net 4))
 (segment (start 122.209999 28.060401) (end 122.209999 28.8925) (width 0.2) (layer "F.Cu") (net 4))
 (via (at 123.444 26.416) (size 0.6) (drill 0.2) (layers "F.Cu" "B.Cu") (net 4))
 (segment (start 123.444 27.5176) (end 123.46 27.5336) (width 0.2) (layer "B.Cu") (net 4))
 (segment (start 123.444 26.416) (end 123.444 27.5176) (width 0.2) (layer "B.Cu") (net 4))
 (segment (start 123.709999 27.568401) (end 123.709999 28.8925) (width 0.2) (layer "F.Cu") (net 3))
 (segment (start 123.948 27.3304) (end 123.709999 27.568401) (width 0.2) (layer "F.Cu") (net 3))
 (segment (start 125.5028 28.288989) (end 125.210001 28.581788) (width 0.2) (layer "F.Cu") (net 6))
 (segment (start 127.1564 27.3304) (end 126.197811 28.288989) (width 0.2) (layer "F.Cu") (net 6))
 (segment (start 125.210001 28.581788) (end 125.210001 28.8925) (width 0.2) (layer "F.Cu") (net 6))
 (segment (start 126.197811 28.288989) (end 125.5028 28.288989) (width 0.2) (layer "F.Cu") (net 6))
 (segment (start 121.288844 31.74563) (end 122.43237 31.74563) (width 0.2) (layer "F.Cu") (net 7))
 (segment (start 120.3452 30.801986) (end 121.288844 31.74563) (width 0.2) (layer "F.Cu") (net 7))
 (segment (start 122.43237 31.74563) (end 122.96 31.218) (width 0.2) (layer "F.Cu") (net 7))
 (segment (start 120.3452 30.228) (end 120.3452 30.801986) (width 0.2) (layer "F.Cu") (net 7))
 (segment (start 122.96 31.218) (end 122.96 30.7975) (width 0.2) (layer "F.Cu") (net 7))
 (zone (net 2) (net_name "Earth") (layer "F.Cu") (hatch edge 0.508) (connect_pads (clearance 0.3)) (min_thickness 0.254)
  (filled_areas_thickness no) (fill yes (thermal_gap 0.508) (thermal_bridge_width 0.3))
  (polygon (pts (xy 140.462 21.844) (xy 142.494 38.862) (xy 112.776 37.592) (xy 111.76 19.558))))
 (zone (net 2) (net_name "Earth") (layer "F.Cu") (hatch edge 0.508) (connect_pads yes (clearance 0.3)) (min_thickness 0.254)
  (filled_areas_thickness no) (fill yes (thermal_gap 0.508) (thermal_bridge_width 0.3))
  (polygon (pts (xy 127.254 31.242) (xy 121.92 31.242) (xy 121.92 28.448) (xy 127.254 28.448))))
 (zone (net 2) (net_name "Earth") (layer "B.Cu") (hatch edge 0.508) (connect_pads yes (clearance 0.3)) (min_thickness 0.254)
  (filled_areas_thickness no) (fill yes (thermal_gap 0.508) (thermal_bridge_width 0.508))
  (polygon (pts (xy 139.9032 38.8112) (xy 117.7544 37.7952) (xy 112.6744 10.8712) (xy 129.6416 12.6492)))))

